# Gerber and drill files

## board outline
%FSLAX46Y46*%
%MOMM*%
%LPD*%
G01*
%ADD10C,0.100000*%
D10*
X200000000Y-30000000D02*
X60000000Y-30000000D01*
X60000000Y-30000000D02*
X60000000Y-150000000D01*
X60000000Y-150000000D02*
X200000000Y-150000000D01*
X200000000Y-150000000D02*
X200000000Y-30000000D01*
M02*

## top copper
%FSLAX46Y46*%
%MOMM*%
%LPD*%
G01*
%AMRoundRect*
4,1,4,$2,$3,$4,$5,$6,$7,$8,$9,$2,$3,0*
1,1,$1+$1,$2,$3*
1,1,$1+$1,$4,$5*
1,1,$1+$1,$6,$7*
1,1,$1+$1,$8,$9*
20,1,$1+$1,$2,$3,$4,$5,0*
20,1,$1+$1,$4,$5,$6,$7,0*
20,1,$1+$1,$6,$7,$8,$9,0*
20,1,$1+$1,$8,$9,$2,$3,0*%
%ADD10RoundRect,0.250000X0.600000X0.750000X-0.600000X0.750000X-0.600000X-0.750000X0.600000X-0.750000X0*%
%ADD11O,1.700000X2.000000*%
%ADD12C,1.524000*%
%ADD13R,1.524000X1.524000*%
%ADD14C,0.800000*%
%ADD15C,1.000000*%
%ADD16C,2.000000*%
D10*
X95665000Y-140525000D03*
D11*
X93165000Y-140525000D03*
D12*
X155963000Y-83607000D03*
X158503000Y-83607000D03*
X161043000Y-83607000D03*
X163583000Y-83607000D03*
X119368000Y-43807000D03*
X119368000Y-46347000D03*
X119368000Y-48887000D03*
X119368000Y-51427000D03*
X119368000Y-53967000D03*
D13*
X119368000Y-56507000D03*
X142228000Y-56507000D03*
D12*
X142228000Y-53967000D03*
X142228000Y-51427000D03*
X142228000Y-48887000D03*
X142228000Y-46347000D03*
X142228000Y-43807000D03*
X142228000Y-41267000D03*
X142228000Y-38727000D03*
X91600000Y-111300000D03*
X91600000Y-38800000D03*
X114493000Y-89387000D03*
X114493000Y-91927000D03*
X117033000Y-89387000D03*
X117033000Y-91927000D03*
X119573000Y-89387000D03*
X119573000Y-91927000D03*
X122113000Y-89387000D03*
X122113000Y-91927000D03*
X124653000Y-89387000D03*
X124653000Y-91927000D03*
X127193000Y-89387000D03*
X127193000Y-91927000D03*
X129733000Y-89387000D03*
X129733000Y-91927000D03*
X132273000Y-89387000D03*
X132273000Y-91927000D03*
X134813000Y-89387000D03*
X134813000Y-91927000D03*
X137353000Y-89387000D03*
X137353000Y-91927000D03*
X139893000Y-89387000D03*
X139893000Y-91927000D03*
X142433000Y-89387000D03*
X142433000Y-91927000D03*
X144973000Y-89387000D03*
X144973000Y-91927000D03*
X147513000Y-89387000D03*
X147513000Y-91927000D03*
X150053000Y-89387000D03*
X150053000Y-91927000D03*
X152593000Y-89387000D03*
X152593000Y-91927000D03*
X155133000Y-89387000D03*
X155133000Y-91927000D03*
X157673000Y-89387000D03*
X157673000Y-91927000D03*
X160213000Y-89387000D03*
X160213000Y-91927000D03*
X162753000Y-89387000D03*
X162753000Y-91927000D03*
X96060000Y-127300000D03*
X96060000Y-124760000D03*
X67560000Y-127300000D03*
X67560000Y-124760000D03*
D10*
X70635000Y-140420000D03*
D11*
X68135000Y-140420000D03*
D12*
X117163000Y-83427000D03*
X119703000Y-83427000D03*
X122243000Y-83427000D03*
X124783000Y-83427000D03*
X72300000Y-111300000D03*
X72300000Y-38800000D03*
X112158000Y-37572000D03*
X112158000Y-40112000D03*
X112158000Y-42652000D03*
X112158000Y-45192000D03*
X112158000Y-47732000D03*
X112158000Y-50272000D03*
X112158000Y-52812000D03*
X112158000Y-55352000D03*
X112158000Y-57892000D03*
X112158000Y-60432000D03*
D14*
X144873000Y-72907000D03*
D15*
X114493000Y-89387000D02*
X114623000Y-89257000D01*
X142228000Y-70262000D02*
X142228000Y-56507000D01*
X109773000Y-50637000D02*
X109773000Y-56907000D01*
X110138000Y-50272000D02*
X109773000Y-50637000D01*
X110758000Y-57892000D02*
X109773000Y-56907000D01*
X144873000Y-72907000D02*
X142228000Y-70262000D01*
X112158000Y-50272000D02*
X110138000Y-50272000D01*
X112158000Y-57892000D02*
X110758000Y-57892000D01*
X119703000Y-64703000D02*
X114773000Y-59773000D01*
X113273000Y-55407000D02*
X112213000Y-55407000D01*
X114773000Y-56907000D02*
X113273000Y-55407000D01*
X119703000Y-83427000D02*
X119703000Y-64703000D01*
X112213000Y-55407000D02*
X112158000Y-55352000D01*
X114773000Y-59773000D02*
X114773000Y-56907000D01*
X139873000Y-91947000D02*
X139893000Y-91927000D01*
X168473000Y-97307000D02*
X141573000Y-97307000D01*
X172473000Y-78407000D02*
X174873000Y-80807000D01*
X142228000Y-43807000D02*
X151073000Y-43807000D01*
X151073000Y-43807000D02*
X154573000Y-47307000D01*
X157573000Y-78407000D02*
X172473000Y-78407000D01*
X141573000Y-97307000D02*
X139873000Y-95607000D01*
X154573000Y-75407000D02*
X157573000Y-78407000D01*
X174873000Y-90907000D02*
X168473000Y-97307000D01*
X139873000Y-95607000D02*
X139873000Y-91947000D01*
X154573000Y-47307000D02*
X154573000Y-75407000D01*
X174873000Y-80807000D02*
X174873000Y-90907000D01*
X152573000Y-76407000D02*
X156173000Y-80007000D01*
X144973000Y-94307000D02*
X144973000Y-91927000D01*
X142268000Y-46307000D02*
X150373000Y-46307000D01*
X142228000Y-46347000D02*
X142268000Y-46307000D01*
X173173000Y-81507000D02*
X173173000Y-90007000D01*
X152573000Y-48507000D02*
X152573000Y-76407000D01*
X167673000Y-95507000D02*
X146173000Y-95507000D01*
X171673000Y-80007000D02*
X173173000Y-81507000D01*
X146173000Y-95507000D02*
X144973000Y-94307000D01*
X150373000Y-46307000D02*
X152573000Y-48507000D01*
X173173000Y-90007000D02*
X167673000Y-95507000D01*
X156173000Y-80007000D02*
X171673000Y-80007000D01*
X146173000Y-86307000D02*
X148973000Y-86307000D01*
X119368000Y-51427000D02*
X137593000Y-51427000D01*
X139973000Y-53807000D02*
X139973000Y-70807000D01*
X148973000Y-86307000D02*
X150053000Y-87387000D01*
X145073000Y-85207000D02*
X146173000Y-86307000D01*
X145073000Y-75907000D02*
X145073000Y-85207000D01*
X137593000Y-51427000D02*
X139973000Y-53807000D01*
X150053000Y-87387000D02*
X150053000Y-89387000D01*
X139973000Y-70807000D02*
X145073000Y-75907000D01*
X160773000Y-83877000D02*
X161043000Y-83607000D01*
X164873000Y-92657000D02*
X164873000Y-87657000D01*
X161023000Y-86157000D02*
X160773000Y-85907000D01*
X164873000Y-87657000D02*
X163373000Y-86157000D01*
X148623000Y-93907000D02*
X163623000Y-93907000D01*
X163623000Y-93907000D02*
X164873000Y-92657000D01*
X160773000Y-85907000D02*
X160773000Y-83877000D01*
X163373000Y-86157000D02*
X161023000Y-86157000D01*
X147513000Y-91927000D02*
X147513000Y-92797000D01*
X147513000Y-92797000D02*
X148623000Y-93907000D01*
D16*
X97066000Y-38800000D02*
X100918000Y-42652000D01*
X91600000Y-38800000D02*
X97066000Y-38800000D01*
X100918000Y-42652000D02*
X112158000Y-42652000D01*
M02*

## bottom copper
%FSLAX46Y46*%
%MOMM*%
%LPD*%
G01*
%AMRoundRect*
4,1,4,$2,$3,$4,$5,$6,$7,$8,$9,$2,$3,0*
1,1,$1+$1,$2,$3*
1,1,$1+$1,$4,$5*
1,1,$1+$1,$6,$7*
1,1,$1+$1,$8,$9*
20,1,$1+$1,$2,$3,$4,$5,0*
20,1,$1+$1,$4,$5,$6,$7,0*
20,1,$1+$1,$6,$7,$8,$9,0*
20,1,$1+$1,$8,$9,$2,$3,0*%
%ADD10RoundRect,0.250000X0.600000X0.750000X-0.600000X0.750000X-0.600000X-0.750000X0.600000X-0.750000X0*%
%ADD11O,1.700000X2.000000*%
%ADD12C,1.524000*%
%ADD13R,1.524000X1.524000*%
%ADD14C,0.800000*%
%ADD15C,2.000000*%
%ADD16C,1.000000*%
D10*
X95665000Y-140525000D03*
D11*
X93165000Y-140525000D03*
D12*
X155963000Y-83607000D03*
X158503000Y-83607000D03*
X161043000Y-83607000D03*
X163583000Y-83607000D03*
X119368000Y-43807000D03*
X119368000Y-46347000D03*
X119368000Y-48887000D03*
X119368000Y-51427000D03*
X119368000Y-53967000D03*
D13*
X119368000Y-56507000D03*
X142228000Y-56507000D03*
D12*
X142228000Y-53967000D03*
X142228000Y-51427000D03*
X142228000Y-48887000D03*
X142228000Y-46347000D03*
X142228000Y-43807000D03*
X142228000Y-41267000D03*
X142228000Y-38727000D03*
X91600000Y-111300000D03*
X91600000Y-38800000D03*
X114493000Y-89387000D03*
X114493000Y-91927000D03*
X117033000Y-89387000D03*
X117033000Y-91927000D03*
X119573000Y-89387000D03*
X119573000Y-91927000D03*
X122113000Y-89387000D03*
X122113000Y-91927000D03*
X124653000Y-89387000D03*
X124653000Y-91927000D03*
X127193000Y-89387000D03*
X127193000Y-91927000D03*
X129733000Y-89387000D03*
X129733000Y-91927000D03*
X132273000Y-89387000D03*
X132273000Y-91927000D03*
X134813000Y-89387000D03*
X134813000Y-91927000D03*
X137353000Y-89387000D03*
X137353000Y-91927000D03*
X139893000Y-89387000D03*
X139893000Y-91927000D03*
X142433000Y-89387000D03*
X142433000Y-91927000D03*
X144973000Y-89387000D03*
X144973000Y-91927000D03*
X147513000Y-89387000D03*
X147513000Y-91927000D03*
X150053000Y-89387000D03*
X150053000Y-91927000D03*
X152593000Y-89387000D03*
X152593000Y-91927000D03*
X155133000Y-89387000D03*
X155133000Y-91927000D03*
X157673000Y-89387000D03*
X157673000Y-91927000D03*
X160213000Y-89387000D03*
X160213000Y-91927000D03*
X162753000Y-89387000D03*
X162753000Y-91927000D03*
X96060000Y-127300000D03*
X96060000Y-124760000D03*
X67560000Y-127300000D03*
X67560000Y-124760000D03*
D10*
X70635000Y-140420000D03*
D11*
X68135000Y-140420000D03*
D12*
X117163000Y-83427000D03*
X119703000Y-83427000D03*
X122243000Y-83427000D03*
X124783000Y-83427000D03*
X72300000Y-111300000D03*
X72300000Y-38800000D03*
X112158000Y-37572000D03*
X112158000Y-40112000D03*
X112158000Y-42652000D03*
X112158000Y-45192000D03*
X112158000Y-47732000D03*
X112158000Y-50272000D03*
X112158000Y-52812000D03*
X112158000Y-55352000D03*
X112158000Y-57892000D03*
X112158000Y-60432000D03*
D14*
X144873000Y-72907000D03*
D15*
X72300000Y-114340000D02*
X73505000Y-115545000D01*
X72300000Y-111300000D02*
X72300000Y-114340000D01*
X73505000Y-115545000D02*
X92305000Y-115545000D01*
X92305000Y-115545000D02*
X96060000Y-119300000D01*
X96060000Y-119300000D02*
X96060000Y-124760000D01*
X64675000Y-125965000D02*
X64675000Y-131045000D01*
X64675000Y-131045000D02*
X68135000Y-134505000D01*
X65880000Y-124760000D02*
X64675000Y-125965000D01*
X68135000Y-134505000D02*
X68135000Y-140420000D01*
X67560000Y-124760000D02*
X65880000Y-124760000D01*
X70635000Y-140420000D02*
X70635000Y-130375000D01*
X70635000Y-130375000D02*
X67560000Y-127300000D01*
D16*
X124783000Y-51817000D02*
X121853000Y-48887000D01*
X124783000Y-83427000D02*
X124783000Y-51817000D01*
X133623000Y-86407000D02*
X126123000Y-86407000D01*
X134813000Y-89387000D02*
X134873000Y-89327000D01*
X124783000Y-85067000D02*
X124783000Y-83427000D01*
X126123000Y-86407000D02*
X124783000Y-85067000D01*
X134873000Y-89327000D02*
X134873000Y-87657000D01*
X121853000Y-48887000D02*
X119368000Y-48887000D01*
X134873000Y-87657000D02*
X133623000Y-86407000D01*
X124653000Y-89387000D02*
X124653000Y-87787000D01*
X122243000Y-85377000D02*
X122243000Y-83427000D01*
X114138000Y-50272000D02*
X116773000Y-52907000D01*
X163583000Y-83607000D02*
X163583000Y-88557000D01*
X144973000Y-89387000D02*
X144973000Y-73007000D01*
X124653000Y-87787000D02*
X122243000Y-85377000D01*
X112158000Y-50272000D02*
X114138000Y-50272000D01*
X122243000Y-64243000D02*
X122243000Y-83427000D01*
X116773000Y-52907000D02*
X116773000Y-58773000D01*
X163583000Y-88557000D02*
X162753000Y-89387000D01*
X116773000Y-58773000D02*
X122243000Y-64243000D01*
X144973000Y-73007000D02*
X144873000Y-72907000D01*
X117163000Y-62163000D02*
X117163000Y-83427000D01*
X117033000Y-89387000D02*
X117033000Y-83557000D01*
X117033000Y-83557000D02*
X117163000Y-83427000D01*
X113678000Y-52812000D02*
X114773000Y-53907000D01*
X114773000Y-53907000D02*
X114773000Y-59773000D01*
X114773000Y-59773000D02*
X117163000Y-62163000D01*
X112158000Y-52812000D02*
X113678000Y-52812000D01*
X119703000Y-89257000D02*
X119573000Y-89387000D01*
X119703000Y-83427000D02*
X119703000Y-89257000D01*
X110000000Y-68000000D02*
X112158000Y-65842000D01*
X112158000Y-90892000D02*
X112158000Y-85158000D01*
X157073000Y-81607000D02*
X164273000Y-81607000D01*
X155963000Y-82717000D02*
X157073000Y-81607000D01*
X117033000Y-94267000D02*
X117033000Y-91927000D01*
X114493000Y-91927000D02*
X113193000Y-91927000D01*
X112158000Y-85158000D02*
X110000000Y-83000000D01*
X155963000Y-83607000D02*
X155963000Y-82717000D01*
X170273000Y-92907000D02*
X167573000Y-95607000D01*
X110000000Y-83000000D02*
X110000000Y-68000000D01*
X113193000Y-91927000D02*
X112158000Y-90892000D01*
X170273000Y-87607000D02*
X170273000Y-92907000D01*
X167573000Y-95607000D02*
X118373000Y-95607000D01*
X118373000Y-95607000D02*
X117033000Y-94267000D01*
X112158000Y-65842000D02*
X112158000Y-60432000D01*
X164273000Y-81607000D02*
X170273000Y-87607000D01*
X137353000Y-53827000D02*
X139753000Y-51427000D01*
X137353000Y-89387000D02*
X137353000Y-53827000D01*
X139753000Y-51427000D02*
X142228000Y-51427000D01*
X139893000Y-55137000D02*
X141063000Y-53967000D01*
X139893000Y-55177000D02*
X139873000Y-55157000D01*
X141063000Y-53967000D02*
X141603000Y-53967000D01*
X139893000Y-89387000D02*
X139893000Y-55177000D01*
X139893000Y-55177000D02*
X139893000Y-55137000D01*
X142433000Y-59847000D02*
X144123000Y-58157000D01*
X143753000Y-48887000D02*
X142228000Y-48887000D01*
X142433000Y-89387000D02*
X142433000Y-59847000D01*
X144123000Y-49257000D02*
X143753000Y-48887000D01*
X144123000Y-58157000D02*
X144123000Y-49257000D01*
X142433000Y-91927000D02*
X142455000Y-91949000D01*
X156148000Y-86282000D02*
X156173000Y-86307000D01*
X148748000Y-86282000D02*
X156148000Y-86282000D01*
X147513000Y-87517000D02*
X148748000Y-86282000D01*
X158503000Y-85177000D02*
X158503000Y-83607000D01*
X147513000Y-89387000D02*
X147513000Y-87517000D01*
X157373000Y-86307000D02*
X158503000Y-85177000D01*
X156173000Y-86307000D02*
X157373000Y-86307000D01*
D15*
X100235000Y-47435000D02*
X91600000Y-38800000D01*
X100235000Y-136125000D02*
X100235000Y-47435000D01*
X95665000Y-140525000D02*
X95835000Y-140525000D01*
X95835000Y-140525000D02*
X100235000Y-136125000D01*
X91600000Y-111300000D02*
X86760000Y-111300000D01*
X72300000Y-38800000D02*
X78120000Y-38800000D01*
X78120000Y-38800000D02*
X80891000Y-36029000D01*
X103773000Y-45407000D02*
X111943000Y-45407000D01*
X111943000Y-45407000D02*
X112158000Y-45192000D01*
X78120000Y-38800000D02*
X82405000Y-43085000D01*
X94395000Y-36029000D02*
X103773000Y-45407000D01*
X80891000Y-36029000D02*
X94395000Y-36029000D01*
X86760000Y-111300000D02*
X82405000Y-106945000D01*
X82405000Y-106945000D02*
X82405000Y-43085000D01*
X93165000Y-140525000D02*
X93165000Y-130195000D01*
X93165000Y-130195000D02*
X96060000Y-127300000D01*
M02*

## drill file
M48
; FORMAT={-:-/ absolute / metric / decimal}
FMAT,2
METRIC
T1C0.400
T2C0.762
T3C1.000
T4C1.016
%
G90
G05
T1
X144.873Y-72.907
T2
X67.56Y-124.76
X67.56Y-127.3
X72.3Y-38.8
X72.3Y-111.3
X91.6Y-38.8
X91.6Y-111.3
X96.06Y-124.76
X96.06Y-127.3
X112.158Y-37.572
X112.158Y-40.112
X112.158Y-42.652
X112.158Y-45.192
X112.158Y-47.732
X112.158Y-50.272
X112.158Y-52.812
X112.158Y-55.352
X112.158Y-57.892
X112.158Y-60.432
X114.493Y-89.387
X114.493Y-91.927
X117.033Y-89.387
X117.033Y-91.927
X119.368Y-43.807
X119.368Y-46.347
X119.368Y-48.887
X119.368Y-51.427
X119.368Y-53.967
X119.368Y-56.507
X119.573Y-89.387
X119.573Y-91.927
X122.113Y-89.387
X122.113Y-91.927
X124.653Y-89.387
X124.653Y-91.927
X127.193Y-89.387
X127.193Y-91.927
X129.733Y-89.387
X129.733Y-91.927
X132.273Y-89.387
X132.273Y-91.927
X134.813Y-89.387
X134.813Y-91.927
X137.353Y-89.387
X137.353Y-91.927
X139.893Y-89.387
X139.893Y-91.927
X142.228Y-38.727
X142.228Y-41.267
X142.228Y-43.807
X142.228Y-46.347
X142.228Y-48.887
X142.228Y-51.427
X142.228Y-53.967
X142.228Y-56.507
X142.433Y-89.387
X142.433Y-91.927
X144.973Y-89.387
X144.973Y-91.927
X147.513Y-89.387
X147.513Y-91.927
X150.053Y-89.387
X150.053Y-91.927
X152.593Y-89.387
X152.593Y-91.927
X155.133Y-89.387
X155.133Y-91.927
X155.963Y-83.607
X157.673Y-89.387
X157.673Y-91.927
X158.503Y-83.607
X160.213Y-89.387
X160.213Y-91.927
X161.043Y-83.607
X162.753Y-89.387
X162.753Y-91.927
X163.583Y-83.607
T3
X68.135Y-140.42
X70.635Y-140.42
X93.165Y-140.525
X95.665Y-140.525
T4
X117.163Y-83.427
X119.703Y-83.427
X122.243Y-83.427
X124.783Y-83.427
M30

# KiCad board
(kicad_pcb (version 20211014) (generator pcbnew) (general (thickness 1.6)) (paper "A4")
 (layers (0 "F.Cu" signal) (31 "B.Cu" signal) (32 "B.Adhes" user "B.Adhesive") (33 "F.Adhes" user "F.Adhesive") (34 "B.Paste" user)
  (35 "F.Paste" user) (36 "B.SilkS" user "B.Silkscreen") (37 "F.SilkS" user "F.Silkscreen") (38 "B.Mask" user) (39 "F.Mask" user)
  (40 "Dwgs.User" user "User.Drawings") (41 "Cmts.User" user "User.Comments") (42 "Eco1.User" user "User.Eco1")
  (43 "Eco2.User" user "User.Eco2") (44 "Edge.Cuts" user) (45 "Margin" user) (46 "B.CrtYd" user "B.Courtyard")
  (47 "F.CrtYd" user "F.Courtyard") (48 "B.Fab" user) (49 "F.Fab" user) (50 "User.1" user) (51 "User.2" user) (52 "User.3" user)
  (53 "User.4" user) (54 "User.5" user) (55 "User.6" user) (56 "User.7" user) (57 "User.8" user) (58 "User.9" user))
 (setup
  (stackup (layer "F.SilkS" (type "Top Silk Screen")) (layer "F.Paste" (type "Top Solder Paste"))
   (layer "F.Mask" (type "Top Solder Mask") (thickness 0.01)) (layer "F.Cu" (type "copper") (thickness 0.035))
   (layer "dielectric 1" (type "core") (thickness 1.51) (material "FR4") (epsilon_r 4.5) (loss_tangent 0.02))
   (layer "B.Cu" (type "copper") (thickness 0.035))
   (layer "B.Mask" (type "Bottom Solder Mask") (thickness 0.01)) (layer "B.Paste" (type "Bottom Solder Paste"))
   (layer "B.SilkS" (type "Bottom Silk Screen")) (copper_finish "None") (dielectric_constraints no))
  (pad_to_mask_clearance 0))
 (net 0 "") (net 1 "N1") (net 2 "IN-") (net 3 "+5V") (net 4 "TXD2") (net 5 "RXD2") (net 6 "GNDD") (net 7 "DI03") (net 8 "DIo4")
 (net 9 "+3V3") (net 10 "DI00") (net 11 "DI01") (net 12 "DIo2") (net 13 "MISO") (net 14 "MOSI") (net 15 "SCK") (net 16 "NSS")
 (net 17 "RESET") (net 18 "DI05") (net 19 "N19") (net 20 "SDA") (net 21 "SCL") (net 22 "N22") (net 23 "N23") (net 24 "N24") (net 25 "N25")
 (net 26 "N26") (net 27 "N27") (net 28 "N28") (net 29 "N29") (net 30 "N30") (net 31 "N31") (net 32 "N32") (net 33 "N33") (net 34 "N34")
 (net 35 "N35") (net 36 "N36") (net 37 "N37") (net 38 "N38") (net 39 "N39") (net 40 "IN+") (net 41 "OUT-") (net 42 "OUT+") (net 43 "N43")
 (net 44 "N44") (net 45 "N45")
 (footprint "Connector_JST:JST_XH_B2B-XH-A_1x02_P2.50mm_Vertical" (layer "F.Cu") (at 95.665 140.525 180)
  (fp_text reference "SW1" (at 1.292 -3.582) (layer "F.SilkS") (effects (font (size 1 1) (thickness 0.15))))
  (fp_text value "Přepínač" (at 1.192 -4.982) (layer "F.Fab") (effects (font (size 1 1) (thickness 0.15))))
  (pad "1" thru_hole roundrect (at 0 0 180) (size 1.7 2) (drill 1) (layers *.Cu *.Mask) (roundrect_rratio 0.1470588235) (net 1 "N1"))
  (pad "2" thru_hole oval (at 2.5 0 180) (size 1.7 2) (drill 1) (layers *.Cu *.Mask) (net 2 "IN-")))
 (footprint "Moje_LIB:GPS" (layer "F.Cu") (at 159.773 85.507 180)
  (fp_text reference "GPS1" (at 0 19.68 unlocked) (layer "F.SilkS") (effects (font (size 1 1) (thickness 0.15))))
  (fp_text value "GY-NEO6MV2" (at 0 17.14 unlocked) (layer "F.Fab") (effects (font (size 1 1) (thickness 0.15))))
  (pad "1" thru_hole circle (at 3.81 1.9) (size 1.524 1.524) (drill 0.762) (layers *.Cu *.Mask) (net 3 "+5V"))
  (pad "2" thru_hole circle (at 1.27 1.9) (size 1.524 1.524) (drill 0.762) (layers *.Cu *.Mask) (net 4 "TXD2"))
  (pad "3" thru_hole circle (at -1.27 1.9) (size 1.524 1.524) (drill 0.762) (layers *.Cu *.Mask) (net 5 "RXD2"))
  (pad "4" thru_hole circle (at -3.81 1.9) (size 1.524 1.524) (drill 0.762) (layers *.Cu *.Mask) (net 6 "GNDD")))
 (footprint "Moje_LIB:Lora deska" (layer "F.Cu") (at 117.368 36.477)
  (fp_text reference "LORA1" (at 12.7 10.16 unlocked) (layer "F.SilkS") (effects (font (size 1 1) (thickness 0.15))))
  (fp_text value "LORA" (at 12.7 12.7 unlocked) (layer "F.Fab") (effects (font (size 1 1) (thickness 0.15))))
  (pad "3" thru_hole circle (at 2 7.33) (size 1.524 1.524) (drill 0.762) (layers *.Cu *.Mask) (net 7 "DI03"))
  (pad "4" thru_hole circle (at 2 9.87) (size 1.524 1.524) (drill 0.762) (layers *.Cu *.Mask) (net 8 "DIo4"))
  (pad "5" thru_hole circle (at 2 12.41) (size 1.524 1.524) (drill 0.762) (layers *.Cu *.Mask) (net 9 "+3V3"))
  (pad "6" thru_hole circle (at 2 14.95) (size 1.524 1.524) (drill 0.762) (layers *.Cu *.Mask) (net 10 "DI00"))
  (pad "7" thru_hole circle (at 2 17.49) (size 1.524 1.524) (drill 0.762) (layers *.Cu *.Mask) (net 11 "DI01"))
  (pad "8" thru_hole rect (at 2 20.03) (size 1.524 1.524) (drill 0.762) (layers *.Cu *.Mask) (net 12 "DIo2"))
  (pad "9" thru_hole rect (at 24.86 20.03) (size 1.524 1.524) (drill 0.762) (layers *.Cu *.Mask) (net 6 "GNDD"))
  (pad "10" thru_hole circle (at 24.86 17.49) (size 1.524 1.524) (drill 0.762) (layers *.Cu *.Mask) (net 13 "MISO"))
  (pad "11" thru_hole circle (at 24.86 14.95) (size 1.524 1.524) (drill 0.762) (layers *.Cu *.Mask) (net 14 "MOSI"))
  (pad "12" thru_hole circle (at 24.86 12.41) (size 1.524 1.524) (drill 0.762) (layers *.Cu *.Mask) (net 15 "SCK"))
  (pad "13" thru_hole circle (at 24.86 9.87) (size 1.524 1.524) (drill 0.762) (layers *.Cu *.Mask) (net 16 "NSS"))
  (pad "14" thru_hole circle (at 24.86 7.33) (size 1.524 1.524) (drill 0.762) (layers *.Cu *.Mask) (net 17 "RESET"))
  (pad "15" thru_hole circle (at 24.86 4.79) (size 1.524 1.524) (drill 0.762) (layers *.Cu *.Mask) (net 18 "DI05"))
  (pad "16" thru_hole circle (at 24.86 2.25) (size 1.524 1.524) (drill 0.762) (layers *.Cu *.Mask) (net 6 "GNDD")))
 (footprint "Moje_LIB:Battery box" (layer "F.Cu") (at 81.95 113.9 90)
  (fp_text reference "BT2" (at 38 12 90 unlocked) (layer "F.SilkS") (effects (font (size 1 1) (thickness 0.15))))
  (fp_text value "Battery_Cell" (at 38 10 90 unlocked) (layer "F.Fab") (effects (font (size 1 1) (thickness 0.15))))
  (pad "1" thru_hole circle (at 2.6 9.65 90) (size 1.524 1.524) (drill 0.762) (layers *.Cu *.Mask) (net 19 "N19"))
  (pad "2" thru_hole circle (at 75.1 9.65 90) (size 1.524 1.524) (drill 0.762) (layers *.Cu *.Mask) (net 1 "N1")))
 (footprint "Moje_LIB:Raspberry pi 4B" (layer "F.Cu") (at 191.123 115.157 -90)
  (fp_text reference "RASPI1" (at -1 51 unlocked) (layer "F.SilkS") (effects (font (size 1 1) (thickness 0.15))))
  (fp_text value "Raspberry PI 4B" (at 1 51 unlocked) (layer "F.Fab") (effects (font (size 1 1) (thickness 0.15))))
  (pad "1" thru_hole circle (at -25.77 76.63) (size 1.524 1.524) (drill 0.762) (layers *.Cu *.Mask) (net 9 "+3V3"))
  (pad "2" thru_hole circle (at -23.23 76.63) (size 1.524 1.524) (drill 0.762) (layers *.Cu *.Mask) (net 3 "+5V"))
  (pad "3" thru_hole circle (at -25.77 74.09) (size 1.524 1.524) (drill 0.762) (layers *.Cu *.Mask) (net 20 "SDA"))
  (pad "4" thru_hole circle (at -23.23 74.09) (size 1.524 1.524) (drill 0.762) (layers *.Cu *.Mask) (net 3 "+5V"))
  (pad "5" thru_hole circle (at -25.77 71.55) (size 1.524 1.524) (drill 0.762) (layers *.Cu *.Mask) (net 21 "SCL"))
  (pad "6" thru_hole circle (at -23.23 71.55) (size 1.524 1.524) (drill 0.762) (layers *.Cu *.Mask) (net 6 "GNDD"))
  (pad "7" thru_hole circle (at -25.77 69.01) (size 1.524 1.524) (drill 0.762) (layers *.Cu *.Mask) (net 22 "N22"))
  (pad "8" thru_hole circle (at -23.23 69.01) (size 1.524 1.524) (drill 0.762) (layers *.Cu *.Mask) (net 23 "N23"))
  (pad "9" thru_hole circle (at -25.77 66.47) (size 1.524 1.524) (drill 0.762) (layers *.Cu *.Mask) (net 6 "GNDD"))
  (pad "10" thru_hole circle (at -23.23 66.47) (size 1.524 1.524) (drill 0.762) (layers *.Cu *.Mask) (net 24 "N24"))
  (pad "11" thru_hole circle (at -25.77 63.93) (size 1.524 1.524) (drill 0.762) (layers *.Cu *.Mask) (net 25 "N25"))
  (pad "12" thru_hole circle (at -23.23 63.93) (size 1.524 1.524) (drill 0.762) (layers *.Cu *.Mask) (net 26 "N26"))
  (pad "13" thru_hole circle (at -25.77 61.39) (size 1.524 1.524) (drill 0.762) (layers *.Cu *.Mask) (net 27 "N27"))
  (pad "14" thru_hole circle (at -23.23 61.39) (size 1.524 1.524) (drill 0.762) (layers *.Cu *.Mask) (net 6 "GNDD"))
  (pad "15" thru_hole circle (at -25.77 58.85) (size 1.524 1.524) (drill 0.762) (layers *.Cu *.Mask) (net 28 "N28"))
  (pad "16" thru_hole circle (at -23.23 58.85) (size 1.524 1.524) (drill 0.762) (layers *.Cu *.Mask) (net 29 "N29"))
  (pad "17" thru_hole circle (at -25.77 56.31) (size 1.524 1.524) (drill 0.762) (layers *.Cu *.Mask) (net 9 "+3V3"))
  (pad "18" thru_hole circle (at -23.23 56.31) (size 1.524 1.524) (drill 0.762) (layers *.Cu *.Mask) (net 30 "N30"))
  (pad "19" thru_hole circle (at -25.77 53.77) (size 1.524 1.524) (drill 0.762) (layers *.Cu *.Mask) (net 14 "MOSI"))
  (pad "20" thru_hole circle (at -23.23 53.77) (size 1.524 1.524) (drill 0.762) (layers *.Cu *.Mask) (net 6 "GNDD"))
  (pad "21" thru_hole circle (at -25.77 51.23) (size 1.524 1.524) (drill 0.762) (layers *.Cu *.Mask) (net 13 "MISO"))
  (pad "22" thru_hole circle (at -23.23 51.23) (size 1.524 1.524) (drill 0.762) (layers *.Cu *.Mask) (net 17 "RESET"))
  (pad "23" thru_hole circle (at -25.77 48.69) (size 1.524 1.524) (drill 0.762) (layers *.Cu *.Mask) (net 15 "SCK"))
  (pad "24" thru_hole circle (at -23.23 48.69) (size 1.524 1.524) (drill 0.762) (layers *.Cu *.Mask) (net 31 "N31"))
  (pad "25" thru_hole circle (at -25.77 46.15) (size 1.524 1.524) (drill 0.762) (layers *.Cu *.Mask) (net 6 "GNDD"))
  (pad "26" thru_hole circle (at -23.23 46.15) (size 1.524 1.524) (drill 0.762) (layers *.Cu *.Mask) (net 16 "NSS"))
  (pad "27" thru_hole circle (at -25.77 43.61) (size 1.524 1.524) (drill 0.762) (layers *.Cu *.Mask) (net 4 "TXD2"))
  (pad "28" thru_hole circle (at -23.23 43.61) (size 1.524 1.524) (drill 0.762) (layers *.Cu *.Mask) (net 5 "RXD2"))
  (pad "29" thru_hole circle (at -25.77 41.07) (size 1.524 1.524) (drill 0.762) (layers *.Cu *.Mask) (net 10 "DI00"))
  (pad "30" thru_hole circle (at -23.23 41.07) (size 1.524 1.524) (drill 0.762) (layers *.Cu *.Mask) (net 6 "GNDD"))
  (pad "31" thru_hole circle (at -25.77 38.53) (size 1.524 1.524) (drill 0.762) (layers *.Cu *.Mask) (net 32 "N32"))
  (pad "32" thru_hole circle (at -23.23 38.53) (size 1.524 1.524) (drill 0.762) (layers *.Cu *.Mask) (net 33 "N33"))
  (pad "33" thru_hole circle (at -25.77 35.99) (size 1.524 1.524) (drill 0.762) (layers *.Cu *.Mask) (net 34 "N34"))
  (pad "34" thru_hole circle (at -23.23 35.99) (size 1.524 1.524) (drill 0.762) (layers *.Cu *.Mask) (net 6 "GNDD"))
  (pad "35" thru_hole circle (at -25.77 33.45) (size 1.524 1.524) (drill 0.762) (layers *.Cu *.Mask) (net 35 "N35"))
  (pad "36" thru_hole circle (at -23.23 33.45) (size 1.524 1.524) (drill 0.762) (layers *.Cu *.Mask) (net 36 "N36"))
  (pad "37" thru_hole circle (at -25.77 30.91) (size 1.524 1.524) (drill 0.762) (layers *.Cu *.Mask) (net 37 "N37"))
  (pad "38" thru_hole circle (at -23.23 30.91) (size 1.524 1.524) (drill 0.762) (layers *.Cu *.Mask) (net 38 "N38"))
  (pad "39" thru_hole circle (at -25.77 28.37) (size 1.524 1.524) (drill 0.762) (layers *.Cu *.Mask) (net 6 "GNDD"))
  (pad "40" thru_hole circle (at -23.23 28.37) (size 1.524 1.524) (drill 0.762) (layers *.Cu *.Mask) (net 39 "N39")))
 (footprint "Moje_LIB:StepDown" (layer "F.Cu") (at 98.56 135.3 180)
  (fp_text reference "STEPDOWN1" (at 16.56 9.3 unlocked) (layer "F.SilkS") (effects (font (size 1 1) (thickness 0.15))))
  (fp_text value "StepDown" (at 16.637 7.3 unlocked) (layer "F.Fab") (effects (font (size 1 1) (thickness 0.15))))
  (pad "1" thru_hole circle (at 2.5 8 180) (size 1.524 1.524) (drill 0.762) (layers *.Cu *.Mask) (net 2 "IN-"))
  (pad "2" thru_hole circle (at 2.5 10.54 180) (size 1.524 1.524) (drill 0.762) (layers *.Cu *.Mask) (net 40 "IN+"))
  (pad "3" thru_hole circle (at 31 8 180) (size 1.524 1.524) (drill 0.762) (layers *.Cu *.Mask) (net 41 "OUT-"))
  (pad "4" thru_hole circle (at 31 10.54 180) (size 1.524 1.524) (drill 0.762) (layers *.Cu *.Mask) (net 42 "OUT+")))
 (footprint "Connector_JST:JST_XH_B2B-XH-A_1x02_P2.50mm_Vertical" (layer "F.Cu") (at 70.635 140.42 180)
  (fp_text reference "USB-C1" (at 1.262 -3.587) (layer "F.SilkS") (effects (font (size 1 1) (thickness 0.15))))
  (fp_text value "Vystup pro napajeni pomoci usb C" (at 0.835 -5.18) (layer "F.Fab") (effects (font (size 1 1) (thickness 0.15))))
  (pad "1" thru_hole roundrect (at 0 0 180) (size 1.7 2) (drill 1) (layers *.Cu *.Mask) (roundrect_rratio 0.1470588235) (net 41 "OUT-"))
  (pad "2" thru_hole oval (at 2.5 0 180) (size 1.7 2) (drill 1) (layers *.Cu *.Mask) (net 42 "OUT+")))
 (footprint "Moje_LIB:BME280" (layer "F.Cu") (at 120.973 63.107)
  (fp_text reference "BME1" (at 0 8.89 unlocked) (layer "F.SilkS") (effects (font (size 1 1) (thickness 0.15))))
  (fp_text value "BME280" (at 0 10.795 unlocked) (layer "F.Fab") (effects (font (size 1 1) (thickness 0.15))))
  (pad "1" thru_hole circle (at -3.81 20.32) (size 1.524 1.524) (drill 1.016) (layers *.Cu *.Mask) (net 20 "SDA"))
  (pad "2" thru_hole circle (at -1.27 20.32) (size 1.524 1.524) (drill 1.016) (layers *.Cu *.Mask) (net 21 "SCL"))
  (pad "3" thru_hole circle (at 1.27 20.32) (size 1.524 1.524) (drill 1.016) (layers *.Cu *.Mask) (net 6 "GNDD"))
  (pad "4" thru_hole circle (at 3.81 20.32) (size 1.524 1.524) (drill 1.016) (layers *.Cu *.Mask) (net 9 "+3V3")))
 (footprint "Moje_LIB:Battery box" (layer "F.Cu") (at 62.65 113.9 90)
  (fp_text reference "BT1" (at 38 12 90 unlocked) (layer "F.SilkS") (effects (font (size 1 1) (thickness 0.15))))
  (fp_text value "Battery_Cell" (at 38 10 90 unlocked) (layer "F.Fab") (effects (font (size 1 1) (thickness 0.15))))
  (pad "1" thru_hole circle (at 2.6 9.65 90) (size 1.524 1.524) (drill 0.762) (layers *.Cu *.Mask) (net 40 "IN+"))
  (pad "2" thru_hole circle (at 75.1 9.65 90) (size 1.524 1.524) (drill 0.762) (layers *.Cu *.Mask) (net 19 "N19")))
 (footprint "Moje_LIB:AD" (layer "F.Cu") (at 113.428 36.002 -90)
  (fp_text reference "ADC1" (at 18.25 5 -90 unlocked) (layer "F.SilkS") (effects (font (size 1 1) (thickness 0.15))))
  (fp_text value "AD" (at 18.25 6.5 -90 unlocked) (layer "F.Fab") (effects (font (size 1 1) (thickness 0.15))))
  (pad "1" thru_hole circle (at 1.57 1.27 270) (size 1.524 1.524) (drill 0.762) (layers *.Cu *.Mask) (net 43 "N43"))
  (pad "2" thru_hole circle (at 4.11 1.27 270) (size 1.524 1.524) (drill 0.762) (layers *.Cu *.Mask) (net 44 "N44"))
  (pad "3" thru_hole circle (at 6.65 1.27 270) (size 1.524 1.524) (drill 0.762) (layers *.Cu *.Mask) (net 1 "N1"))
  (pad "4" thru_hole circle (at 9.19 1.27 270) (size 1.524 1.524) (drill 0.762) (layers *.Cu *.Mask) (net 19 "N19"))
  (pad "5" thru_hole circle (at 11.73 1.27 270) (size 1.524 1.524) (drill 0.762) (layers *.Cu *.Mask) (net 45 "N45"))
  (pad "6" thru_hole circle (at 14.27 1.27 270) (size 1.524 1.524) (drill 0.762) (layers *.Cu *.Mask) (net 6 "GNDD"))
  (pad "7" thru_hole circle (at 16.81 1.27 270) (size 1.524 1.524) (drill 0.762) (layers *.Cu *.Mask) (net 20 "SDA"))
  (pad "8" thru_hole circle (at 19.35 1.27 270) (size 1.524 1.524) (drill 0.762) (layers *.Cu *.Mask) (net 21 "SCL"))
  (pad "9" thru_hole circle (at 21.89 1.27 270) (size 1.524 1.524) (drill 0.762) (layers *.Cu *.Mask) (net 6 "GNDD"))
  (pad "10" thru_hole circle (at 24.43 1.27 270) (size 1.524 1.524) (drill 0.762) (layers *.Cu *.Mask) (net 3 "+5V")))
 (gr_line (start 200 30) (end 60 30) (layer "Edge.Cuts") (width 0.1))
 (gr_line (start 60 30) (end 60 150) (layer "Edge.Cuts") (width 0.1))
 (gr_line (start 60 150) (end 200 150) (layer "Edge.Cuts") (width 0.1))
 (gr_line (start 200 150) (end 200 30) (layer "Edge.Cuts") (width 0.1))
 (segment (start 72.3 114.34) (end 73.505 115.545) (width 2) (layer "B.Cu") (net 40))
 (segment (start 72.3 111.3) (end 72.3 114.34) (width 2) (layer "B.Cu") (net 40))
 (segment (start 73.505 115.545) (end 92.305 115.545) (width 2) (layer "B.Cu") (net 40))
 (segment (start 92.305 115.545) (end 96.06 119.3) (width 2) (layer "B.Cu") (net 40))
 (segment (start 96.06 119.3) (end 96.06 124.76) (width 2) (layer "B.Cu") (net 40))
 (segment (start 64.675 125.965) (end 64.675 131.045) (width 2) (layer "B.Cu") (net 42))
 (segment (start 64.675 131.045) (end 68.135 134.505) (width 2) (layer "B.Cu") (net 42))
 (segment (start 65.88 124.76) (end 64.675 125.965) (width 2) (layer "B.Cu") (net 42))
 (segment (start 68.135 134.505) (end 68.135 140.42) (width 2) (layer "B.Cu") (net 42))
 (segment (start 67.56 124.76) (end 65.88 124.76) (width 2) (layer "B.Cu") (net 42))
 (segment (start 70.635 140.42) (end 70.635 130.375) (width 2) (layer "B.Cu") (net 41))
 (segment (start 70.635 130.375) (end 67.56 127.3) (width 2) (layer "B.Cu") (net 41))
 (segment (start 114.493 89.387) (end 114.623 89.257) (width 1) (layer "F.Cu") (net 9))
 (segment (start 124.783 51.817) (end 121.853 48.887) (width 1) (layer "B.Cu") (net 9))
 (segment (start 124.783 83.427) (end 124.783 51.817) (width 1) (layer "B.Cu") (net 9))
 (segment (start 133.623 86.407) (end 126.123 86.407) (width 1) (layer "B.Cu") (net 9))
 (segment (start 134.813 89.387) (end 134.873 89.327) (width 1) (layer "B.Cu") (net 9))
 (segment (start 124.783 85.067) (end 124.783 83.427) (width 1) (layer "B.Cu") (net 9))
 (segment (start 126.123 86.407) (end 124.783 85.067) (width 1) (layer "B.Cu") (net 9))
 (segment (start 134.873 89.327) (end 134.873 87.657) (width 1) (layer "B.Cu") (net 9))
 (segment (start 121.853 48.887) (end 119.368 48.887) (width 1) (layer "B.Cu") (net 9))
 (segment (start 134.873 87.657) (end 133.623 86.407) (width 1) (layer "B.Cu") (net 9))
 (segment (start 142.228 70.262) (end 142.228 56.507) (width 1) (layer "F.Cu") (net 6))
 (segment (start 109.773 50.637) (end 109.773 56.907) (width 1) (layer "F.Cu") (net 6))
 (segment (start 110.138 50.272) (end 109.773 50.637) (width 1) (layer "F.Cu") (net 6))
 (segment (start 110.758 57.892) (end 109.773 56.907) (width 1) (layer "F.Cu") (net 6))
 (segment (start 144.873 72.907) (end 142.228 70.262) (width 1) (layer "F.Cu") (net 6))
 (segment (start 112.158 50.272) (end 110.138 50.272) (width 1) (layer "F.Cu") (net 6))
 (segment (start 112.158 57.892) (end 110.758 57.892) (width 1) (layer "F.Cu") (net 6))
 (via (at 144.873 72.907) (size 0.8) (drill 0.4) (layers "F.Cu" "B.Cu") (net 6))
 (segment (start 124.653 89.387) (end 124.653 87.787) (width 1) (layer "B.Cu") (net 6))
 (segment (start 122.243 85.377) (end 122.243 83.427) (width 1) (layer "B.Cu") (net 6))
 (segment (start 114.138 50.272) (end 116.773 52.907) (width 1) (layer "B.Cu") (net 6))
 (segment (start 163.583 83.607) (end 163.583 88.557) (width 1) (layer "B.Cu") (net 6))
 (segment (start 144.973 89.387) (end 144.973 73.007) (width 1) (layer "B.Cu") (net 6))
 (segment (start 124.653 87.787) (end 122.243 85.377) (width 1) (layer "B.Cu") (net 6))
 (segment (start 112.158 50.272) (end 114.138 50.272) (width 1) (layer "B.Cu") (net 6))
 (segment (start 122.243 64.243) (end 122.243 83.427) (width 1) (layer "B.Cu") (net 6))
 (segment (start 116.773 52.907) (end 116.773 58.773) (width 1) (layer "B.Cu") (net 6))
 (segment (start 163.583 88.557) (end 162.753 89.387) (width 1) (layer "B.Cu") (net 6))
 (segment (start 116.773 58.773) (end 122.243 64.243) (width 1) (layer "B.Cu") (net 6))
 (segment (start 144.973 73.007) (end 144.873 72.907) (width 1) (layer "B.Cu") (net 6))
 (segment (start 117.163 62.163) (end 117.163 83.427) (width 1) (layer "B.Cu") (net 20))
 (segment (start 117.033 89.387) (end 117.033 83.557) (width 1) (layer "B.Cu") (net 20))
 (segment (start 117.033 83.557) (end 117.163 83.427) (width 1) (layer "B.Cu") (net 20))
 (segment (start 113.678 52.812) (end 114.773 53.907) (width 1) (layer "B.Cu") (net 20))
 (segment (start 114.773 53.907) (end 114.773 59.773) (width 1) (layer "B.Cu") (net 20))
 (segment (start 114.773 59.773) (end 117.163 62.163) (width 1) (layer "B.Cu") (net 20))
 (segment (start 112.158 52.812) (end 113.678 52.812) (width 1) (layer "B.Cu") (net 20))
 (segment (start 119.703 64.703) (end 114.773 59.773) (width 1) (layer "F.Cu") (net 21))
 (segment (start 113.273 55.407) (end 112.213 55.407) (width 1) (layer "F.Cu") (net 21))
 (segment (start 114.773 56.907) (end 113.273 55.407) (width 1) (layer "F.Cu") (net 21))
 (segment (start 119.703 83.427) (end 119.703 64.703) (width 1) (layer "F.Cu") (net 21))
 (segment (start 112.213 55.407) (end 112.158 55.352) (width 1) (layer "F.Cu") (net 21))
 (segment (start 114.773 59.773) (end 114.773 56.907) (width 1) (layer "F.Cu") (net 21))
 (segment (start 119.703 89.257) (end 119.573 89.387) (width 1) (layer "B.Cu") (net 21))
 (segment (start 119.703 83.427) (end 119.703 89.257) (width 1) (layer "B.Cu") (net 21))
 (segment (start 110 68) (end 112.158 65.842) (width 1) (layer "B.Cu") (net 3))
 (segment (start 112.158 90.892) (end 112.158 85.158) (width 1) (layer "B.Cu") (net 3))
 (segment (start 157.073 81.607) (end 164.273 81.607) (width 1) (layer "B.Cu") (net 3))
 (segment (start 155.963 82.717) (end 157.073 81.607) (width 1) (layer "B.Cu") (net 3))
 (segment (start 117.033 94.267) (end 117.033 91.927) (width 1) (layer "B.Cu") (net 3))
 (segment (start 114.493 91.927) (end 113.193 91.927) (width 1) (layer "B.Cu") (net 3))
 (segment (start 112.158 85.158) (end 110 83) (width 1) (layer "B.Cu") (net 3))
 (segment (start 155.963 83.607) (end 155.963 82.717) (width 1) (layer "B.Cu") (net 3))
 (segment (start 170.273 92.907) (end 167.573 95.607) (width 1) (layer "B.Cu") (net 3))
 (segment (start 110 83) (end 110 68) (width 1) (layer "B.Cu") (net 3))
 (segment (start 113.193 91.927) (end 112.158 90.892) (width 1) (layer "B.Cu") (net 3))
 (segment (start 170.273 87.607) (end 170.273 92.907) (width 1) (layer "B.Cu") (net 3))
 (segment (start 167.573 95.607) (end 118.373 95.607) (width 1) (layer "B.Cu") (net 3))
 (segment (start 118.373 95.607) (end 117.033 94.267) (width 1) (layer "B.Cu") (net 3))
 (segment (start 112.158 65.842) (end 112.158 60.432) (width 1) (layer "B.Cu") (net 3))
 (segment (start 164.273 81.607) (end 170.273 87.607) (width 1) (layer "B.Cu") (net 3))
 (segment (start 137.353 53.827) (end 139.753 51.427) (width 1) (layer "B.Cu") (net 14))
 (segment (start 137.353 89.387) (end 137.353 53.827) (width 1) (layer "B.Cu") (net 14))
 (segment (start 139.753 51.427) (end 142.228 51.427) (width 1) (layer "B.Cu") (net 14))
 (segment (start 139.893 55.137) (end 141.063 53.967) (width 1) (layer "B.Cu") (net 13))
 (segment (start 139.893 55.177) (end 139.873 55.157) (width 1) (layer "B.Cu") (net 13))
 (segment (start 141.063 53.967) (end 141.603 53.967) (width 1) (layer "B.Cu") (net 13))
 (segment (start 139.893 89.387) (end 139.893 55.177) (width 1) (layer "B.Cu") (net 13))
 (segment (start 139.893 55.177) (end 139.893 55.137) (width 1) (layer "B.Cu") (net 13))
 (segment (start 142.433 59.847) (end 144.123 58.157) (width 1) (layer "B.Cu") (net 15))
 (segment (start 143.753 48.887) (end 142.228 48.887) (width 1) (layer "B.Cu") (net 15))
 (segment (start 142.433 89.387) (end 142.433 59.847) (width 1) (layer "B.Cu") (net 15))
 (segment (start 144.123 49.257) (end 143.753 48.887) (width 1) (layer "B.Cu") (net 15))
 (segment (start 144.123 58.157) (end 144.123 49.257) (width 1) (layer "B.Cu") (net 15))
 (segment (start 142.433 91.927) (end 142.455 91.949) (width 1) (layer "B.Cu") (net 31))
 (segment (start 139.873 91.947) (end 139.893 91.927) (width 1) (layer "F.Cu") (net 17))
 (segment (start 168.473 97.307) (end 141.573 97.307) (width 1) (layer "F.Cu") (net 17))
 (segment (start 172.473 78.407) (end 174.873 80.807) (width 1) (layer "F.Cu") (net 17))
 (segment (start 142.228 43.807) (end 151.073 43.807) (width 1) (layer "F.Cu") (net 17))
 (segment (start 151.073 43.807) (end 154.573 47.307) (width 1) (layer "F.Cu") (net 17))
 (segment (start 157.573 78.407) (end 172.473 78.407) (width 1) (layer "F.Cu") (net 17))
 (segment (start 141.573 97.307) (end 139.873 95.607) (width 1) (layer "F.Cu") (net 17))
 (segment (start 154.573 75.407) (end 157.573 78.407) (width 1) (layer "F.Cu") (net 17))
 (segment (start 174.873 90.907) (end 168.473 97.307) (width 1) (layer "F.Cu") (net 17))
 (segment (start 139.873 95.607) (end 139.873 91.947) (width 1) (layer "F.Cu") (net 17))
 (segment (start 154.573 47.307) (end 154.573 75.407) (width 1) (layer "F.Cu") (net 17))
 (segment (start 174.873 80.807) (end 174.873 90.907) (width 1) (layer "F.Cu") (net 17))
 (segment (start 152.573 76.407) (end 156.173 80.007) (width 1) (layer "F.Cu") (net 16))
 (segment (start 144.973 94.307) (end 144.973 91.927) (width 1) (layer "F.Cu") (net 16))
 (segment (start 142.268 46.307) (end 150.373 46.307) (width 1) (layer "F.Cu") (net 16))
 (segment (start 142.228 46.347) (end 142.268 46.307) (width 1) (layer "F.Cu") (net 16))
 (segment (start 173.173 81.507) (end 173.173 90.007) (width 1) (layer "F.Cu") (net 16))
 (segment (start 152.573 48.507) (end 152.573 76.407) (width 1) (layer "F.Cu") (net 16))
 (segment (start 167.673 95.507) (end 146.173 95.507) (width 1) (layer "F.Cu") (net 16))
 (segment (start 171.673 80.007) (end 173.173 81.507) (width 1) (layer "F.Cu") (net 16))
 (segment (start 146.173 95.507) (end 144.973 94.307) (width 1) (layer "F.Cu") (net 16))
 (segment (start 150.373 46.307) (end 152.573 48.507) (width 1) (layer "F.Cu") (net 16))
 (segment (start 173.173 90.007) (end 167.673 95.507) (width 1) (layer "F.Cu") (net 16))
 (segment (start 156.173 80.007) (end 171.673 80.007) (width 1) (layer "F.Cu") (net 16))
 (segment (start 146.173 86.307) (end 148.973 86.307) (width 1) (layer "F.Cu") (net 10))
 (segment (start 119.368 51.427) (end 137.593 51.427) (width 1) (layer "F.Cu") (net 10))
 (segment (start 139.973 53.807) (end 139.973 70.807) (width 1) (layer "F.Cu") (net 10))
 (segment (start 148.973 86.307) (end 150.053 87.387) (width 1) (layer "F.Cu") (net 10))
 (segment (start 145.073 85.207) (end 146.173 86.307) (width 1) (layer "F.Cu") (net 10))
 (segment (start 145.073 75.907) (end 145.073 85.207) (width 1) (layer "F.Cu") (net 10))
 (segment (start 137.593 51.427) (end 139.973 53.807) (width 1) (layer "F.Cu") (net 10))
 (segment (start 150.053 87.387) (end 150.053 89.387) (width 1) (layer "F.Cu") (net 10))
 (segment (start 139.973 70.807) (end 145.073 75.907) (width 1) (layer "F.Cu") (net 10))
 (segment (start 160.773 83.877) (end 161.043 83.607) (width 1) (layer "F.Cu") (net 5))
 (segment (start 164.873 92.657) (end 164.873 87.657) (width 1) (layer "F.Cu") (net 5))
 (segment (start 161.023 86.157) (end 160.773 85.907) (width 1) (layer "F.Cu") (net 5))
 (segment (start 164.873 87.657) (end 163.373 86.157) (width 1) (layer "F.Cu") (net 5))
 (segment (start 148.623 93.907) (end 163.623 93.907) (width 1) (layer "F.Cu") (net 5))
 (segment (start 163.623 93.907) (end 164.873 92.657) (width 1) (layer "F.Cu") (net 5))
 (segment (start 160.773 85.907) (end 160.773 83.877) (width 1) (layer "F.Cu") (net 5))
 (segment (start 163.373 86.157) (end 161.023 86.157) (width 1) (layer "F.Cu") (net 5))
 (segment (start 147.513 91.927) (end 147.513 92.797) (width 1) (layer "F.Cu") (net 5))
 (segment (start 147.513 92.797) (end 148.623 93.907) (width 1) (layer "F.Cu") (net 5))
 (segment (start 156.148 86.282) (end 156.173 86.307) (width 1) (layer "B.Cu") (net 4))
 (segment (start 148.748 86.282) (end 156.148 86.282) (width 1) (layer "B.Cu") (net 4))
 (segment (start 147.513 87.517) (end 148.748 86.282) (width 1) (layer "B.Cu") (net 4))
 (segment (start 158.503 85.177) (end 158.503 83.607) (width 1) (layer "B.Cu") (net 4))
 (segment (start 147.513 89.387) (end 147.513 87.517) (width 1) (layer "B.Cu") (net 4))
 (segment (start 157.373 86.307) (end 158.503 85.177) (width 1) (layer "B.Cu") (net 4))
 (segment (start 156.173 86.307) (end 157.373 86.307) (width 1) (layer "B.Cu") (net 4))
 (segment (start 97.066 38.8) (end 100.918 42.652) (width 2) (layer "F.Cu") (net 1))
 (segment (start 91.6 38.8) (end 97.066 38.8) (width 2) (layer "F.Cu") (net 1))
 (segment (start 100.918 42.652) (end 112.158 42.652) (width 2) (layer "F.Cu") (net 1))
 (segment (start 100.235 47.435) (end 91.6 38.8) (width 2) (layer "B.Cu") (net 1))
 (segment (start 100.235 136.125) (end 100.235 47.435) (width 2) (layer "B.Cu") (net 1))
 (segment (start 95.665 140.525) (end 95.835 140.525) (width 2) (layer "B.Cu") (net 1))
 (segment (start 95.835 140.525) (end 100.235 136.125) (width 2) (layer "B.Cu") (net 1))
 (segment (start 91.6 111.3) (end 86.76 111.3) (width 2) (layer "B.Cu") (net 19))
 (segment (start 72.3 38.8) (end 78.12 38.8) (width 2) (layer "B.Cu") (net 19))
 (segment (start 78.12 38.8) (end 80.891 36.029) (width 2) (layer "B.Cu") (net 19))
 (segment (start 103.773 45.407) (end 111.943 45.407) (width 2) (layer "B.Cu") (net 19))
 (segment (start 111.943 45.407) (end 112.158 45.192) (width 2) (layer "B.Cu") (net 19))
 (segment (start 78.12 38.8) (end 82.405 43.085) (width 2) (layer "B.Cu") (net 19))
 (segment (start 94.395 36.029) (end 103.773 45.407) (width 2) (layer "B.Cu") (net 19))
 (segment (start 80.891 36.029) (end 94.395 36.029) (width 2) (layer "B.Cu") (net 19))
 (segment (start 86.76 111.3) (end 82.405 106.945) (width 2) (layer "B.Cu") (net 19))
 (segment (start 82.405 106.945) (end 82.405 43.085) (width 2) (layer "B.Cu") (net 19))
 (segment (start 93.165 140.525) (end 93.165 130.195) (width 2) (layer "B.Cu") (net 2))
 (segment (start 93.165 130.195) (end 96.06 127.3) (width 2) (layer "B.Cu") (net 2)))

